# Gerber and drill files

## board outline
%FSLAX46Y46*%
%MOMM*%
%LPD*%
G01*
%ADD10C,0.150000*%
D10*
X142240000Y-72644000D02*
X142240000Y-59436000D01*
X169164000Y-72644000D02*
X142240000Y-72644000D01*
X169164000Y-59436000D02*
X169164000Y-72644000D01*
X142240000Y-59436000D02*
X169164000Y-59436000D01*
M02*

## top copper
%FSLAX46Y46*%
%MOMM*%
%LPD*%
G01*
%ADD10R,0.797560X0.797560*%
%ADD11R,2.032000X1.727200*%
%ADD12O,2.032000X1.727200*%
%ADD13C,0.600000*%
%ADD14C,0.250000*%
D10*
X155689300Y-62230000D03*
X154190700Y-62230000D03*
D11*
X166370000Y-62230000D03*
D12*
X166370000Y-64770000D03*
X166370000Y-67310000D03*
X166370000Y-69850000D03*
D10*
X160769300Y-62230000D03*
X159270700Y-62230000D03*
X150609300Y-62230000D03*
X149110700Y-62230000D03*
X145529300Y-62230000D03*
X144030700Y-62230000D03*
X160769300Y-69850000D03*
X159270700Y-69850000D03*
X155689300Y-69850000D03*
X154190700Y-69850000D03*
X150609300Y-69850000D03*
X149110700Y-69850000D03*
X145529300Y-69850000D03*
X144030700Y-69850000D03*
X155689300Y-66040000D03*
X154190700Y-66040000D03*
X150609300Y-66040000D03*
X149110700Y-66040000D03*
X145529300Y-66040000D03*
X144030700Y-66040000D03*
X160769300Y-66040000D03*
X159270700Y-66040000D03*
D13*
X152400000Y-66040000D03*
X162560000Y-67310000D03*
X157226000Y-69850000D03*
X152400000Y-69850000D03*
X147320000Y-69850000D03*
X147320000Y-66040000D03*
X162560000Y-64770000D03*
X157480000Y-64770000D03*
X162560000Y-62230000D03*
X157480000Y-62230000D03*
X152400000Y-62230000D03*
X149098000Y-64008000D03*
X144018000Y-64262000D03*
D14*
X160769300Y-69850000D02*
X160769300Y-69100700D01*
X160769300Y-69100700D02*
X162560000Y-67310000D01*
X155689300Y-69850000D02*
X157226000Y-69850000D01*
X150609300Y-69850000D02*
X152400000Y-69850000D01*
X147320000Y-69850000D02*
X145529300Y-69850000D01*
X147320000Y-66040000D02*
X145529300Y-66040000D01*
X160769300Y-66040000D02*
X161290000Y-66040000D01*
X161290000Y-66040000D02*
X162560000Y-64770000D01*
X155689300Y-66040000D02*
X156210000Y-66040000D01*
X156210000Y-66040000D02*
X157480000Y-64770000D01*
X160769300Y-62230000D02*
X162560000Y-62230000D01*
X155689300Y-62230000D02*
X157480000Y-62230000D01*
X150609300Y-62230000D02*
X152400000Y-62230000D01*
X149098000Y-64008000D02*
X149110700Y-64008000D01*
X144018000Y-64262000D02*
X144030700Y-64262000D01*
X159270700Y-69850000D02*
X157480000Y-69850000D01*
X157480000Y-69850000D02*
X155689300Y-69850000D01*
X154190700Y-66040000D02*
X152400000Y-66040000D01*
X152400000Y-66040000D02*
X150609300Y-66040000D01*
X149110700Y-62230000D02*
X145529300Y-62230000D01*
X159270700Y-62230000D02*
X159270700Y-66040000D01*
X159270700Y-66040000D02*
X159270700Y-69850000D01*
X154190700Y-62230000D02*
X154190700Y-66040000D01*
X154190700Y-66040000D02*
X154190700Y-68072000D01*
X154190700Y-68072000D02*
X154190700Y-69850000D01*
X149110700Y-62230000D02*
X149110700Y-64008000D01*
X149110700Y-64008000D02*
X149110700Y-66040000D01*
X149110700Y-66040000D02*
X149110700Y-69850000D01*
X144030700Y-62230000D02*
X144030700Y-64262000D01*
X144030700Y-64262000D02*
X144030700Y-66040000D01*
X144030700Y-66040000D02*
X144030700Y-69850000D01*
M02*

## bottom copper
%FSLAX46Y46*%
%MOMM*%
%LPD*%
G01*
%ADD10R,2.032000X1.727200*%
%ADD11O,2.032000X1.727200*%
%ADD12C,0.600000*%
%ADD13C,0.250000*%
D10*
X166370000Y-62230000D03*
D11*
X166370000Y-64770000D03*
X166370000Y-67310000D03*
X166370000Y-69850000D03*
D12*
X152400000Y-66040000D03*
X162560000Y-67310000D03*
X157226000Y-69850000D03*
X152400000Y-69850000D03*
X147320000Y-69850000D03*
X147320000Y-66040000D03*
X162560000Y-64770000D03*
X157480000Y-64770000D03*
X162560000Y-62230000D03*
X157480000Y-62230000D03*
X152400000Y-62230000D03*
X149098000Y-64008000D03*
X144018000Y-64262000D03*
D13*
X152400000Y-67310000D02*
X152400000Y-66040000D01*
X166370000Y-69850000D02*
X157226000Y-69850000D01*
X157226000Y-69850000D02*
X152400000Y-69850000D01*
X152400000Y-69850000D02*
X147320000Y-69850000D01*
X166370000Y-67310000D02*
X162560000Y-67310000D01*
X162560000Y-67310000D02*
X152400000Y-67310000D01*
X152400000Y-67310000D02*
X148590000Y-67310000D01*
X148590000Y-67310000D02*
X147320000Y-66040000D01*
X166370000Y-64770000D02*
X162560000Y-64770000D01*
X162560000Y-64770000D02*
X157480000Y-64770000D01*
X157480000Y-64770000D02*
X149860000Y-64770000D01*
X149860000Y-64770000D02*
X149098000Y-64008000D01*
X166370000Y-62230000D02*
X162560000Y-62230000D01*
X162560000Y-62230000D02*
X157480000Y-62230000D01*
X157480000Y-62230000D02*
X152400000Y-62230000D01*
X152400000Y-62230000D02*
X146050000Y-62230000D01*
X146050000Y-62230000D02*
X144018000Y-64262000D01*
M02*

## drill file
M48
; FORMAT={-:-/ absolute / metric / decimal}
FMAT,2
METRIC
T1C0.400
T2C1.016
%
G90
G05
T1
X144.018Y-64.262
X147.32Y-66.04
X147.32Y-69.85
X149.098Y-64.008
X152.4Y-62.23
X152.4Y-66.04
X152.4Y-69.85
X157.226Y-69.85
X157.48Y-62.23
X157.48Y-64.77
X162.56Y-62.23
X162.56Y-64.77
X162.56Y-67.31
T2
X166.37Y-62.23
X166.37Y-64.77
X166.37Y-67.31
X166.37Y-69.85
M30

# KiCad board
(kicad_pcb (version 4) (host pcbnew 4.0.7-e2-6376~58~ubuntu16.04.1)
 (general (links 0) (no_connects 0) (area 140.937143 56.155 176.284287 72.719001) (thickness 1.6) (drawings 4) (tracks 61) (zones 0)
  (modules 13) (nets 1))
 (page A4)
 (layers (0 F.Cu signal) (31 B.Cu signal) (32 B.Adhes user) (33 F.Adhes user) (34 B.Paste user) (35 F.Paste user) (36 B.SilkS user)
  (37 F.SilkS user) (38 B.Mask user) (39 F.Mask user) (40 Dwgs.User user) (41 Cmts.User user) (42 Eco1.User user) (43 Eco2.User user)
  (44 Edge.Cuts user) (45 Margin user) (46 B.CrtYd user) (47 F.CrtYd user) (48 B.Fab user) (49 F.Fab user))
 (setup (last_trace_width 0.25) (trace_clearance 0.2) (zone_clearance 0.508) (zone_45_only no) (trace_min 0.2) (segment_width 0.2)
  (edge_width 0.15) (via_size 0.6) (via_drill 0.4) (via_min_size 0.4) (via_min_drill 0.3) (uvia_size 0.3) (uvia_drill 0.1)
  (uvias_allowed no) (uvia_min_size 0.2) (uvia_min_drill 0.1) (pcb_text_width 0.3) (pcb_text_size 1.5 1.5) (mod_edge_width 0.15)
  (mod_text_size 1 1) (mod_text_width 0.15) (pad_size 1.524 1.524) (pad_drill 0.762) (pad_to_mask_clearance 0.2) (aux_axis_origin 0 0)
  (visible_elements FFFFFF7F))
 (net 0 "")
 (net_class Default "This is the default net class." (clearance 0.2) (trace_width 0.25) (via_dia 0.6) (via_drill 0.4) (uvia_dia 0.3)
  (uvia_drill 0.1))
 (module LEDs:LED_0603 (layer F.Cu) (at 154.94 62.23)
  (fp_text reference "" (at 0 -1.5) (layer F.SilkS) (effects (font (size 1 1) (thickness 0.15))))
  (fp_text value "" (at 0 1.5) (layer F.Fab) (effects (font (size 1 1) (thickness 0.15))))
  (pad 2 smd rect (at 0.7493 0 180) (size 0.79756 0.79756) (layers F.Cu F.Paste F.Mask))
  (pad 1 smd rect (at -0.7493 0 180) (size 0.79756 0.79756) (layers F.Cu F.Paste F.Mask)))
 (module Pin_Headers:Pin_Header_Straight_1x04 (layer F.Cu) (at 166.37 62.23)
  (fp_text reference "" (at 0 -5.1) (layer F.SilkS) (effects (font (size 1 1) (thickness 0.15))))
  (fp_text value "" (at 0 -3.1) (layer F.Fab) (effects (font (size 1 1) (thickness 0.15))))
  (pad 1 thru_hole rect (at 0 0) (size 2.032 1.7272) (drill 1.016) (layers *.Cu *.Mask F.SilkS))
  (pad 2 thru_hole oval (at 0 2.54) (size 2.032 1.7272) (drill 1.016) (layers *.Cu *.Mask F.SilkS))
  (pad 3 thru_hole oval (at 0 5.08) (size 2.032 1.7272) (drill 1.016) (layers *.Cu *.Mask F.SilkS))
  (pad 4 thru_hole oval (at 0 7.62) (size 2.032 1.7272) (drill 1.016) (layers *.Cu *.Mask F.SilkS)))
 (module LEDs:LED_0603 (layer F.Cu) (at 160.02 62.23)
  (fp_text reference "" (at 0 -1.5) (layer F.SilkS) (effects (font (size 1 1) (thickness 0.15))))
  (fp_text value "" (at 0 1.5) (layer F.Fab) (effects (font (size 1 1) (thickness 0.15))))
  (pad 2 smd rect (at 0.7493 0 180) (size 0.79756 0.79756) (layers F.Cu F.Paste F.Mask))
  (pad 1 smd rect (at -0.7493 0 180) (size 0.79756 0.79756) (layers F.Cu F.Paste F.Mask)))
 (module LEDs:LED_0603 (layer F.Cu) (at 149.86 62.23)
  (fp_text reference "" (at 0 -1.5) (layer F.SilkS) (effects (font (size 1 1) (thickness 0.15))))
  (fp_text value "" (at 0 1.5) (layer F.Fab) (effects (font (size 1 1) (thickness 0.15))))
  (pad 2 smd rect (at 0.7493 0 180) (size 0.79756 0.79756) (layers F.Cu F.Paste F.Mask))
  (pad 1 smd rect (at -0.7493 0 180) (size 0.79756 0.79756) (layers F.Cu F.Paste F.Mask)))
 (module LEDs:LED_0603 (layer F.Cu) (at 144.78 62.23)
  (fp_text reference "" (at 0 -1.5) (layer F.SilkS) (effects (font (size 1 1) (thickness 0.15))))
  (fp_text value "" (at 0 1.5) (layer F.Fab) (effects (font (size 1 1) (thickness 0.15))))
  (pad 2 smd rect (at 0.7493 0 180) (size 0.79756 0.79756) (layers F.Cu F.Paste F.Mask))
  (pad 1 smd rect (at -0.7493 0 180) (size 0.79756 0.79756) (layers F.Cu F.Paste F.Mask)))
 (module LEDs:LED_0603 (layer F.Cu) (at 160.02 69.85)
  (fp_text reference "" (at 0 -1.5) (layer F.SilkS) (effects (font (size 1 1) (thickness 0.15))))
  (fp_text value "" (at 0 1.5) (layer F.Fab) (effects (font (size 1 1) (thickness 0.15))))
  (pad 2 smd rect (at 0.7493 0 180) (size 0.79756 0.79756) (layers F.Cu F.Paste F.Mask))
  (pad 1 smd rect (at -0.7493 0 180) (size 0.79756 0.79756) (layers F.Cu F.Paste F.Mask)))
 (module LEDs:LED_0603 (layer F.Cu) (at 154.94 69.85)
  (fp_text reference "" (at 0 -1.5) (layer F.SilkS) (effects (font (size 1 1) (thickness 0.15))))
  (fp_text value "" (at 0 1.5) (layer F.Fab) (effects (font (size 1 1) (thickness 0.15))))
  (pad 2 smd rect (at 0.7493 0 180) (size 0.79756 0.79756) (layers F.Cu F.Paste F.Mask))
  (pad 1 smd rect (at -0.7493 0 180) (size 0.79756 0.79756) (layers F.Cu F.Paste F.Mask)))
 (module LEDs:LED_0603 (layer F.Cu) (at 149.86 69.85)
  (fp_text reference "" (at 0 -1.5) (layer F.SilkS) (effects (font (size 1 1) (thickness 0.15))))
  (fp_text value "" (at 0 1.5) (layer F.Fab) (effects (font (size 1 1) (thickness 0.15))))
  (pad 2 smd rect (at 0.7493 0 180) (size 0.79756 0.79756) (layers F.Cu F.Paste F.Mask))
  (pad 1 smd rect (at -0.7493 0 180) (size 0.79756 0.79756) (layers F.Cu F.Paste F.Mask)))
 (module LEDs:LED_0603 (layer F.Cu) (at 144.78 69.85)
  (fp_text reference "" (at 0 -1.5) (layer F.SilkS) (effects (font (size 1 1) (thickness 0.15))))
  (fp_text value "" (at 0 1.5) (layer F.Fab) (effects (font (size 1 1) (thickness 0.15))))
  (pad 2 smd rect (at 0.7493 0 180) (size 0.79756 0.79756) (layers F.Cu F.Paste F.Mask))
  (pad 1 smd rect (at -0.7493 0 180) (size 0.79756 0.79756) (layers F.Cu F.Paste F.Mask)))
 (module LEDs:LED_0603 (layer F.Cu) (at 154.94 66.04)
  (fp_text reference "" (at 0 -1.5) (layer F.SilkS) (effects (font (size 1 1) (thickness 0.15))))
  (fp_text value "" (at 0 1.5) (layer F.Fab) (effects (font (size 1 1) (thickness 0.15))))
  (pad 2 smd rect (at 0.7493 0 180) (size 0.79756 0.79756) (layers F.Cu F.Paste F.Mask))
  (pad 1 smd rect (at -0.7493 0 180) (size 0.79756 0.79756) (layers F.Cu F.Paste F.Mask)))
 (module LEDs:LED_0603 (layer F.Cu) (at 149.86 66.04)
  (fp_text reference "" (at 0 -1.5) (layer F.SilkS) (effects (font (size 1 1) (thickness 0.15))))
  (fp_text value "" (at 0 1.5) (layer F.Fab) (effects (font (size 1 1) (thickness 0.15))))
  (pad 2 smd rect (at 0.7493 0 180) (size 0.79756 0.79756) (layers F.Cu F.Paste F.Mask))
  (pad 1 smd rect (at -0.7493 0 180) (size 0.79756 0.79756) (layers F.Cu F.Paste F.Mask)))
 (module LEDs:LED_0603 (layer F.Cu) (at 144.78 66.04)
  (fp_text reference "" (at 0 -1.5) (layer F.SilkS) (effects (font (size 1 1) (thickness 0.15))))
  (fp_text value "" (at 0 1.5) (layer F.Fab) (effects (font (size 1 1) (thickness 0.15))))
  (pad 2 smd rect (at 0.7493 0 180) (size 0.79756 0.79756) (layers F.Cu F.Paste F.Mask))
  (pad 1 smd rect (at -0.7493 0 180) (size 0.79756 0.79756) (layers F.Cu F.Paste F.Mask)))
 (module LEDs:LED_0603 (layer F.Cu) (at 160.02 66.04)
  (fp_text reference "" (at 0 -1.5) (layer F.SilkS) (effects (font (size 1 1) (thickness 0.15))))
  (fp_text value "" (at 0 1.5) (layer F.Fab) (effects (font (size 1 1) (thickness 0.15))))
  (pad 2 smd rect (at 0.7493 0 180) (size 0.79756 0.79756) (layers F.Cu F.Paste F.Mask))
  (pad 1 smd rect (at -0.7493 0 180) (size 0.79756 0.79756) (layers F.Cu F.Paste F.Mask)))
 (gr_line (start 142.24 72.644) (end 142.24 59.436) (angle 90) (layer Edge.Cuts) (width 0.15))
 (gr_line (start 169.164 72.644) (end 142.24 72.644) (angle 90) (layer Edge.Cuts) (width 0.15))
 (gr_line (start 169.164 59.436) (end 169.164 72.644) (angle 90) (layer Edge.Cuts) (width 0.15))
 (gr_line (start 142.24 59.436) (end 169.164 59.436) (angle 90) (layer Edge.Cuts) (width 0.15))
 (segment (start 152.4 67.31) (end 152.4 66.04) (width 0.25) (layer B.Cu) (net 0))
 (via (at 152.4 66.04) (size 0.6) (drill 0.4) (layers F.Cu B.Cu) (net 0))
 (segment (start 160.7693 69.85) (end 160.7693 69.1007) (width 0.25) (layer F.Cu) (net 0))
 (via (at 162.56 67.31) (size 0.6) (drill 0.4) (layers F.Cu B.Cu) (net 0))
 (segment (start 160.7693 69.1007) (end 162.56 67.31) (width 0.25) (layer F.Cu) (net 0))
 (segment (start 155.6893 69.85) (end 157.226 69.85) (width 0.25) (layer F.Cu) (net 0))
 (via (at 157.226 69.85) (size 0.6) (drill 0.4) (layers F.Cu B.Cu) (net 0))
 (segment (start 150.6093 69.85) (end 152.4 69.85) (width 0.25) (layer F.Cu) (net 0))
 (via (at 152.4 69.85) (size 0.6) (drill 0.4) (layers F.Cu B.Cu) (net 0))
 (segment (start 166.37 69.85) (end 157.226 69.85) (width 0.25) (layer B.Cu) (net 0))
 (segment (start 157.226 69.85) (end 152.4 69.85) (width 0.25) (layer B.Cu) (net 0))
 (segment (start 152.4 69.85) (end 147.32 69.85) (width 0.25) (layer B.Cu) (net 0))
 (segment (start 147.32 69.85) (end 145.5293 69.85) (width 0.25) (layer F.Cu) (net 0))
 (via (at 147.32 69.85) (size 0.6) (drill 0.4) (layers F.Cu B.Cu) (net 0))
 (segment (start 166.37 67.31) (end 162.56 67.31) (width 0.25) (layer B.Cu) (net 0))
 (segment (start 162.56 67.31) (end 152.4 67.31) (width 0.25) (layer B.Cu) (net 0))
 (segment (start 152.4 67.31) (end 148.59 67.31) (width 0.25) (layer B.Cu) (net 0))
 (segment (start 147.32 66.04) (end 145.5293 66.04) (width 0.25) (layer F.Cu) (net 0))
 (via (at 147.32 66.04) (size 0.6) (drill 0.4) (layers F.Cu B.Cu) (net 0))
 (segment (start 148.59 67.31) (end 147.32 66.04) (width 0.25) (layer B.Cu) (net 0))
 (segment (start 160.7693 66.04) (end 161.29 66.04) (width 0.25) (layer F.Cu) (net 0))
 (via (at 162.56 64.77) (size 0.6) (drill 0.4) (layers F.Cu B.Cu) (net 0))
 (segment (start 161.29 66.04) (end 162.56 64.77) (width 0.25) (layer F.Cu) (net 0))
 (segment (start 155.6893 66.04) (end 156.21 66.04) (width 0.25) (layer F.Cu) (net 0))
 (via (at 157.48 64.77) (size 0.6) (drill 0.4) (layers F.Cu B.Cu) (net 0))
 (segment (start 156.21 66.04) (end 157.48 64.77) (width 0.25) (layer F.Cu) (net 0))
 (segment (start 160.7693 62.23) (end 162.56 62.23) (width 0.25) (layer F.Cu) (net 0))
 (via (at 162.56 62.23) (size 0.6) (drill 0.4) (layers F.Cu B.Cu) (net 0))
 (segment (start 155.6893 62.23) (end 157.48 62.23) (width 0.25) (layer F.Cu) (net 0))
 (via (at 157.48 62.23) (size 0.6) (drill 0.4) (layers F.Cu B.Cu) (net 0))
 (segment (start 150.6093 62.23) (end 152.4 62.23) (width 0.25) (layer F.Cu) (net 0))
 (via (at 152.4 62.23) (size 0.6) (drill 0.4) (layers F.Cu B.Cu) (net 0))
 (segment (start 166.37 64.77) (end 162.56 64.77) (width 0.25) (layer B.Cu) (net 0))
 (segment (start 162.56 64.77) (end 157.48 64.77) (width 0.25) (layer B.Cu) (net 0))
 (segment (start 157.48 64.77) (end 149.86 64.77) (width 0.25) (layer B.Cu) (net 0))
 (segment (start 149.098 64.008) (end 149.1107 64.008) (width 0.25) (layer F.Cu) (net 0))
 (via (at 149.098 64.008) (size 0.6) (drill 0.4) (layers F.Cu B.Cu) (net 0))
 (segment (start 149.86 64.77) (end 149.098 64.008) (width 0.25) (layer B.Cu) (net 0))
 (segment (start 166.37 62.23) (end 162.56 62.23) (width 0.25) (layer B.Cu) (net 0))
 (segment (start 162.56 62.23) (end 157.48 62.23) (width 0.25) (layer B.Cu) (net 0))
 (segment (start 157.48 62.23) (end 152.4 62.23) (width 0.25) (layer B.Cu) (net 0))
 (segment (start 152.4 62.23) (end 146.05 62.23) (width 0.25) (layer B.Cu) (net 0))
 (segment (start 144.018 64.262) (end 144.0307 64.262) (width 0.25) (layer F.Cu) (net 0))
 (via (at 144.018 64.262) (size 0.6) (drill 0.4) (layers F.Cu B.Cu) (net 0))
 (segment (start 146.05 62.23) (end 144.018 64.262) (width 0.25) (layer B.Cu) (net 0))
 (segment (start 159.2707 69.85) (end 157.48 69.85) (width 0.25) (layer F.Cu) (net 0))
 (segment (start 157.48 69.85) (end 155.6893 69.85) (width 0.25) (layer F.Cu) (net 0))
 (segment (start 154.1907 66.04) (end 152.4 66.04) (width 0.25) (layer F.Cu) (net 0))
 (segment (start 152.4 66.04) (end 150.6093 66.04) (width 0.25) (layer F.Cu) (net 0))
 (segment (start 149.1107 62.23) (end 145.5293 62.23) (width 0.25) (layer F.Cu) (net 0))
 (segment (start 159.2707 62.23) (end 159.2707 66.04) (width 0.25) (layer F.Cu) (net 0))
 (segment (start 159.2707 66.04) (end 159.2707 69.85) (width 0.25) (layer F.Cu) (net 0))
 (segment (start 154.1907 62.23) (end 154.1907 66.04) (width 0.25) (layer F.Cu) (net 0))
 (segment (start 154.1907 66.04) (end 154.1907 68.072) (width 0.25) (layer F.Cu) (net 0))
 (segment (start 154.1907 68.072) (end 154.1907 69.85) (width 0.25) (layer F.Cu) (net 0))
 (segment (start 149.1107 62.23) (end 149.1107 64.008) (width 0.25) (layer F.Cu) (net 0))
 (segment (start 149.1107 64.008) (end 149.1107 66.04) (width 0.25) (layer F.Cu) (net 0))
 (segment (start 149.1107 66.04) (end 149.1107 69.85) (width 0.25) (layer F.Cu) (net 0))
 (segment (start 144.0307 62.23) (end 144.0307 64.262) (width 0.25) (layer F.Cu) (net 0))
 (segment (start 144.0307 64.262) (end 144.0307 66.04) (width 0.25) (layer F.Cu) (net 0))
 (segment (start 144.0307 66.04) (end 144.0307 69.85) (width 0.25) (layer F.Cu) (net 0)))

